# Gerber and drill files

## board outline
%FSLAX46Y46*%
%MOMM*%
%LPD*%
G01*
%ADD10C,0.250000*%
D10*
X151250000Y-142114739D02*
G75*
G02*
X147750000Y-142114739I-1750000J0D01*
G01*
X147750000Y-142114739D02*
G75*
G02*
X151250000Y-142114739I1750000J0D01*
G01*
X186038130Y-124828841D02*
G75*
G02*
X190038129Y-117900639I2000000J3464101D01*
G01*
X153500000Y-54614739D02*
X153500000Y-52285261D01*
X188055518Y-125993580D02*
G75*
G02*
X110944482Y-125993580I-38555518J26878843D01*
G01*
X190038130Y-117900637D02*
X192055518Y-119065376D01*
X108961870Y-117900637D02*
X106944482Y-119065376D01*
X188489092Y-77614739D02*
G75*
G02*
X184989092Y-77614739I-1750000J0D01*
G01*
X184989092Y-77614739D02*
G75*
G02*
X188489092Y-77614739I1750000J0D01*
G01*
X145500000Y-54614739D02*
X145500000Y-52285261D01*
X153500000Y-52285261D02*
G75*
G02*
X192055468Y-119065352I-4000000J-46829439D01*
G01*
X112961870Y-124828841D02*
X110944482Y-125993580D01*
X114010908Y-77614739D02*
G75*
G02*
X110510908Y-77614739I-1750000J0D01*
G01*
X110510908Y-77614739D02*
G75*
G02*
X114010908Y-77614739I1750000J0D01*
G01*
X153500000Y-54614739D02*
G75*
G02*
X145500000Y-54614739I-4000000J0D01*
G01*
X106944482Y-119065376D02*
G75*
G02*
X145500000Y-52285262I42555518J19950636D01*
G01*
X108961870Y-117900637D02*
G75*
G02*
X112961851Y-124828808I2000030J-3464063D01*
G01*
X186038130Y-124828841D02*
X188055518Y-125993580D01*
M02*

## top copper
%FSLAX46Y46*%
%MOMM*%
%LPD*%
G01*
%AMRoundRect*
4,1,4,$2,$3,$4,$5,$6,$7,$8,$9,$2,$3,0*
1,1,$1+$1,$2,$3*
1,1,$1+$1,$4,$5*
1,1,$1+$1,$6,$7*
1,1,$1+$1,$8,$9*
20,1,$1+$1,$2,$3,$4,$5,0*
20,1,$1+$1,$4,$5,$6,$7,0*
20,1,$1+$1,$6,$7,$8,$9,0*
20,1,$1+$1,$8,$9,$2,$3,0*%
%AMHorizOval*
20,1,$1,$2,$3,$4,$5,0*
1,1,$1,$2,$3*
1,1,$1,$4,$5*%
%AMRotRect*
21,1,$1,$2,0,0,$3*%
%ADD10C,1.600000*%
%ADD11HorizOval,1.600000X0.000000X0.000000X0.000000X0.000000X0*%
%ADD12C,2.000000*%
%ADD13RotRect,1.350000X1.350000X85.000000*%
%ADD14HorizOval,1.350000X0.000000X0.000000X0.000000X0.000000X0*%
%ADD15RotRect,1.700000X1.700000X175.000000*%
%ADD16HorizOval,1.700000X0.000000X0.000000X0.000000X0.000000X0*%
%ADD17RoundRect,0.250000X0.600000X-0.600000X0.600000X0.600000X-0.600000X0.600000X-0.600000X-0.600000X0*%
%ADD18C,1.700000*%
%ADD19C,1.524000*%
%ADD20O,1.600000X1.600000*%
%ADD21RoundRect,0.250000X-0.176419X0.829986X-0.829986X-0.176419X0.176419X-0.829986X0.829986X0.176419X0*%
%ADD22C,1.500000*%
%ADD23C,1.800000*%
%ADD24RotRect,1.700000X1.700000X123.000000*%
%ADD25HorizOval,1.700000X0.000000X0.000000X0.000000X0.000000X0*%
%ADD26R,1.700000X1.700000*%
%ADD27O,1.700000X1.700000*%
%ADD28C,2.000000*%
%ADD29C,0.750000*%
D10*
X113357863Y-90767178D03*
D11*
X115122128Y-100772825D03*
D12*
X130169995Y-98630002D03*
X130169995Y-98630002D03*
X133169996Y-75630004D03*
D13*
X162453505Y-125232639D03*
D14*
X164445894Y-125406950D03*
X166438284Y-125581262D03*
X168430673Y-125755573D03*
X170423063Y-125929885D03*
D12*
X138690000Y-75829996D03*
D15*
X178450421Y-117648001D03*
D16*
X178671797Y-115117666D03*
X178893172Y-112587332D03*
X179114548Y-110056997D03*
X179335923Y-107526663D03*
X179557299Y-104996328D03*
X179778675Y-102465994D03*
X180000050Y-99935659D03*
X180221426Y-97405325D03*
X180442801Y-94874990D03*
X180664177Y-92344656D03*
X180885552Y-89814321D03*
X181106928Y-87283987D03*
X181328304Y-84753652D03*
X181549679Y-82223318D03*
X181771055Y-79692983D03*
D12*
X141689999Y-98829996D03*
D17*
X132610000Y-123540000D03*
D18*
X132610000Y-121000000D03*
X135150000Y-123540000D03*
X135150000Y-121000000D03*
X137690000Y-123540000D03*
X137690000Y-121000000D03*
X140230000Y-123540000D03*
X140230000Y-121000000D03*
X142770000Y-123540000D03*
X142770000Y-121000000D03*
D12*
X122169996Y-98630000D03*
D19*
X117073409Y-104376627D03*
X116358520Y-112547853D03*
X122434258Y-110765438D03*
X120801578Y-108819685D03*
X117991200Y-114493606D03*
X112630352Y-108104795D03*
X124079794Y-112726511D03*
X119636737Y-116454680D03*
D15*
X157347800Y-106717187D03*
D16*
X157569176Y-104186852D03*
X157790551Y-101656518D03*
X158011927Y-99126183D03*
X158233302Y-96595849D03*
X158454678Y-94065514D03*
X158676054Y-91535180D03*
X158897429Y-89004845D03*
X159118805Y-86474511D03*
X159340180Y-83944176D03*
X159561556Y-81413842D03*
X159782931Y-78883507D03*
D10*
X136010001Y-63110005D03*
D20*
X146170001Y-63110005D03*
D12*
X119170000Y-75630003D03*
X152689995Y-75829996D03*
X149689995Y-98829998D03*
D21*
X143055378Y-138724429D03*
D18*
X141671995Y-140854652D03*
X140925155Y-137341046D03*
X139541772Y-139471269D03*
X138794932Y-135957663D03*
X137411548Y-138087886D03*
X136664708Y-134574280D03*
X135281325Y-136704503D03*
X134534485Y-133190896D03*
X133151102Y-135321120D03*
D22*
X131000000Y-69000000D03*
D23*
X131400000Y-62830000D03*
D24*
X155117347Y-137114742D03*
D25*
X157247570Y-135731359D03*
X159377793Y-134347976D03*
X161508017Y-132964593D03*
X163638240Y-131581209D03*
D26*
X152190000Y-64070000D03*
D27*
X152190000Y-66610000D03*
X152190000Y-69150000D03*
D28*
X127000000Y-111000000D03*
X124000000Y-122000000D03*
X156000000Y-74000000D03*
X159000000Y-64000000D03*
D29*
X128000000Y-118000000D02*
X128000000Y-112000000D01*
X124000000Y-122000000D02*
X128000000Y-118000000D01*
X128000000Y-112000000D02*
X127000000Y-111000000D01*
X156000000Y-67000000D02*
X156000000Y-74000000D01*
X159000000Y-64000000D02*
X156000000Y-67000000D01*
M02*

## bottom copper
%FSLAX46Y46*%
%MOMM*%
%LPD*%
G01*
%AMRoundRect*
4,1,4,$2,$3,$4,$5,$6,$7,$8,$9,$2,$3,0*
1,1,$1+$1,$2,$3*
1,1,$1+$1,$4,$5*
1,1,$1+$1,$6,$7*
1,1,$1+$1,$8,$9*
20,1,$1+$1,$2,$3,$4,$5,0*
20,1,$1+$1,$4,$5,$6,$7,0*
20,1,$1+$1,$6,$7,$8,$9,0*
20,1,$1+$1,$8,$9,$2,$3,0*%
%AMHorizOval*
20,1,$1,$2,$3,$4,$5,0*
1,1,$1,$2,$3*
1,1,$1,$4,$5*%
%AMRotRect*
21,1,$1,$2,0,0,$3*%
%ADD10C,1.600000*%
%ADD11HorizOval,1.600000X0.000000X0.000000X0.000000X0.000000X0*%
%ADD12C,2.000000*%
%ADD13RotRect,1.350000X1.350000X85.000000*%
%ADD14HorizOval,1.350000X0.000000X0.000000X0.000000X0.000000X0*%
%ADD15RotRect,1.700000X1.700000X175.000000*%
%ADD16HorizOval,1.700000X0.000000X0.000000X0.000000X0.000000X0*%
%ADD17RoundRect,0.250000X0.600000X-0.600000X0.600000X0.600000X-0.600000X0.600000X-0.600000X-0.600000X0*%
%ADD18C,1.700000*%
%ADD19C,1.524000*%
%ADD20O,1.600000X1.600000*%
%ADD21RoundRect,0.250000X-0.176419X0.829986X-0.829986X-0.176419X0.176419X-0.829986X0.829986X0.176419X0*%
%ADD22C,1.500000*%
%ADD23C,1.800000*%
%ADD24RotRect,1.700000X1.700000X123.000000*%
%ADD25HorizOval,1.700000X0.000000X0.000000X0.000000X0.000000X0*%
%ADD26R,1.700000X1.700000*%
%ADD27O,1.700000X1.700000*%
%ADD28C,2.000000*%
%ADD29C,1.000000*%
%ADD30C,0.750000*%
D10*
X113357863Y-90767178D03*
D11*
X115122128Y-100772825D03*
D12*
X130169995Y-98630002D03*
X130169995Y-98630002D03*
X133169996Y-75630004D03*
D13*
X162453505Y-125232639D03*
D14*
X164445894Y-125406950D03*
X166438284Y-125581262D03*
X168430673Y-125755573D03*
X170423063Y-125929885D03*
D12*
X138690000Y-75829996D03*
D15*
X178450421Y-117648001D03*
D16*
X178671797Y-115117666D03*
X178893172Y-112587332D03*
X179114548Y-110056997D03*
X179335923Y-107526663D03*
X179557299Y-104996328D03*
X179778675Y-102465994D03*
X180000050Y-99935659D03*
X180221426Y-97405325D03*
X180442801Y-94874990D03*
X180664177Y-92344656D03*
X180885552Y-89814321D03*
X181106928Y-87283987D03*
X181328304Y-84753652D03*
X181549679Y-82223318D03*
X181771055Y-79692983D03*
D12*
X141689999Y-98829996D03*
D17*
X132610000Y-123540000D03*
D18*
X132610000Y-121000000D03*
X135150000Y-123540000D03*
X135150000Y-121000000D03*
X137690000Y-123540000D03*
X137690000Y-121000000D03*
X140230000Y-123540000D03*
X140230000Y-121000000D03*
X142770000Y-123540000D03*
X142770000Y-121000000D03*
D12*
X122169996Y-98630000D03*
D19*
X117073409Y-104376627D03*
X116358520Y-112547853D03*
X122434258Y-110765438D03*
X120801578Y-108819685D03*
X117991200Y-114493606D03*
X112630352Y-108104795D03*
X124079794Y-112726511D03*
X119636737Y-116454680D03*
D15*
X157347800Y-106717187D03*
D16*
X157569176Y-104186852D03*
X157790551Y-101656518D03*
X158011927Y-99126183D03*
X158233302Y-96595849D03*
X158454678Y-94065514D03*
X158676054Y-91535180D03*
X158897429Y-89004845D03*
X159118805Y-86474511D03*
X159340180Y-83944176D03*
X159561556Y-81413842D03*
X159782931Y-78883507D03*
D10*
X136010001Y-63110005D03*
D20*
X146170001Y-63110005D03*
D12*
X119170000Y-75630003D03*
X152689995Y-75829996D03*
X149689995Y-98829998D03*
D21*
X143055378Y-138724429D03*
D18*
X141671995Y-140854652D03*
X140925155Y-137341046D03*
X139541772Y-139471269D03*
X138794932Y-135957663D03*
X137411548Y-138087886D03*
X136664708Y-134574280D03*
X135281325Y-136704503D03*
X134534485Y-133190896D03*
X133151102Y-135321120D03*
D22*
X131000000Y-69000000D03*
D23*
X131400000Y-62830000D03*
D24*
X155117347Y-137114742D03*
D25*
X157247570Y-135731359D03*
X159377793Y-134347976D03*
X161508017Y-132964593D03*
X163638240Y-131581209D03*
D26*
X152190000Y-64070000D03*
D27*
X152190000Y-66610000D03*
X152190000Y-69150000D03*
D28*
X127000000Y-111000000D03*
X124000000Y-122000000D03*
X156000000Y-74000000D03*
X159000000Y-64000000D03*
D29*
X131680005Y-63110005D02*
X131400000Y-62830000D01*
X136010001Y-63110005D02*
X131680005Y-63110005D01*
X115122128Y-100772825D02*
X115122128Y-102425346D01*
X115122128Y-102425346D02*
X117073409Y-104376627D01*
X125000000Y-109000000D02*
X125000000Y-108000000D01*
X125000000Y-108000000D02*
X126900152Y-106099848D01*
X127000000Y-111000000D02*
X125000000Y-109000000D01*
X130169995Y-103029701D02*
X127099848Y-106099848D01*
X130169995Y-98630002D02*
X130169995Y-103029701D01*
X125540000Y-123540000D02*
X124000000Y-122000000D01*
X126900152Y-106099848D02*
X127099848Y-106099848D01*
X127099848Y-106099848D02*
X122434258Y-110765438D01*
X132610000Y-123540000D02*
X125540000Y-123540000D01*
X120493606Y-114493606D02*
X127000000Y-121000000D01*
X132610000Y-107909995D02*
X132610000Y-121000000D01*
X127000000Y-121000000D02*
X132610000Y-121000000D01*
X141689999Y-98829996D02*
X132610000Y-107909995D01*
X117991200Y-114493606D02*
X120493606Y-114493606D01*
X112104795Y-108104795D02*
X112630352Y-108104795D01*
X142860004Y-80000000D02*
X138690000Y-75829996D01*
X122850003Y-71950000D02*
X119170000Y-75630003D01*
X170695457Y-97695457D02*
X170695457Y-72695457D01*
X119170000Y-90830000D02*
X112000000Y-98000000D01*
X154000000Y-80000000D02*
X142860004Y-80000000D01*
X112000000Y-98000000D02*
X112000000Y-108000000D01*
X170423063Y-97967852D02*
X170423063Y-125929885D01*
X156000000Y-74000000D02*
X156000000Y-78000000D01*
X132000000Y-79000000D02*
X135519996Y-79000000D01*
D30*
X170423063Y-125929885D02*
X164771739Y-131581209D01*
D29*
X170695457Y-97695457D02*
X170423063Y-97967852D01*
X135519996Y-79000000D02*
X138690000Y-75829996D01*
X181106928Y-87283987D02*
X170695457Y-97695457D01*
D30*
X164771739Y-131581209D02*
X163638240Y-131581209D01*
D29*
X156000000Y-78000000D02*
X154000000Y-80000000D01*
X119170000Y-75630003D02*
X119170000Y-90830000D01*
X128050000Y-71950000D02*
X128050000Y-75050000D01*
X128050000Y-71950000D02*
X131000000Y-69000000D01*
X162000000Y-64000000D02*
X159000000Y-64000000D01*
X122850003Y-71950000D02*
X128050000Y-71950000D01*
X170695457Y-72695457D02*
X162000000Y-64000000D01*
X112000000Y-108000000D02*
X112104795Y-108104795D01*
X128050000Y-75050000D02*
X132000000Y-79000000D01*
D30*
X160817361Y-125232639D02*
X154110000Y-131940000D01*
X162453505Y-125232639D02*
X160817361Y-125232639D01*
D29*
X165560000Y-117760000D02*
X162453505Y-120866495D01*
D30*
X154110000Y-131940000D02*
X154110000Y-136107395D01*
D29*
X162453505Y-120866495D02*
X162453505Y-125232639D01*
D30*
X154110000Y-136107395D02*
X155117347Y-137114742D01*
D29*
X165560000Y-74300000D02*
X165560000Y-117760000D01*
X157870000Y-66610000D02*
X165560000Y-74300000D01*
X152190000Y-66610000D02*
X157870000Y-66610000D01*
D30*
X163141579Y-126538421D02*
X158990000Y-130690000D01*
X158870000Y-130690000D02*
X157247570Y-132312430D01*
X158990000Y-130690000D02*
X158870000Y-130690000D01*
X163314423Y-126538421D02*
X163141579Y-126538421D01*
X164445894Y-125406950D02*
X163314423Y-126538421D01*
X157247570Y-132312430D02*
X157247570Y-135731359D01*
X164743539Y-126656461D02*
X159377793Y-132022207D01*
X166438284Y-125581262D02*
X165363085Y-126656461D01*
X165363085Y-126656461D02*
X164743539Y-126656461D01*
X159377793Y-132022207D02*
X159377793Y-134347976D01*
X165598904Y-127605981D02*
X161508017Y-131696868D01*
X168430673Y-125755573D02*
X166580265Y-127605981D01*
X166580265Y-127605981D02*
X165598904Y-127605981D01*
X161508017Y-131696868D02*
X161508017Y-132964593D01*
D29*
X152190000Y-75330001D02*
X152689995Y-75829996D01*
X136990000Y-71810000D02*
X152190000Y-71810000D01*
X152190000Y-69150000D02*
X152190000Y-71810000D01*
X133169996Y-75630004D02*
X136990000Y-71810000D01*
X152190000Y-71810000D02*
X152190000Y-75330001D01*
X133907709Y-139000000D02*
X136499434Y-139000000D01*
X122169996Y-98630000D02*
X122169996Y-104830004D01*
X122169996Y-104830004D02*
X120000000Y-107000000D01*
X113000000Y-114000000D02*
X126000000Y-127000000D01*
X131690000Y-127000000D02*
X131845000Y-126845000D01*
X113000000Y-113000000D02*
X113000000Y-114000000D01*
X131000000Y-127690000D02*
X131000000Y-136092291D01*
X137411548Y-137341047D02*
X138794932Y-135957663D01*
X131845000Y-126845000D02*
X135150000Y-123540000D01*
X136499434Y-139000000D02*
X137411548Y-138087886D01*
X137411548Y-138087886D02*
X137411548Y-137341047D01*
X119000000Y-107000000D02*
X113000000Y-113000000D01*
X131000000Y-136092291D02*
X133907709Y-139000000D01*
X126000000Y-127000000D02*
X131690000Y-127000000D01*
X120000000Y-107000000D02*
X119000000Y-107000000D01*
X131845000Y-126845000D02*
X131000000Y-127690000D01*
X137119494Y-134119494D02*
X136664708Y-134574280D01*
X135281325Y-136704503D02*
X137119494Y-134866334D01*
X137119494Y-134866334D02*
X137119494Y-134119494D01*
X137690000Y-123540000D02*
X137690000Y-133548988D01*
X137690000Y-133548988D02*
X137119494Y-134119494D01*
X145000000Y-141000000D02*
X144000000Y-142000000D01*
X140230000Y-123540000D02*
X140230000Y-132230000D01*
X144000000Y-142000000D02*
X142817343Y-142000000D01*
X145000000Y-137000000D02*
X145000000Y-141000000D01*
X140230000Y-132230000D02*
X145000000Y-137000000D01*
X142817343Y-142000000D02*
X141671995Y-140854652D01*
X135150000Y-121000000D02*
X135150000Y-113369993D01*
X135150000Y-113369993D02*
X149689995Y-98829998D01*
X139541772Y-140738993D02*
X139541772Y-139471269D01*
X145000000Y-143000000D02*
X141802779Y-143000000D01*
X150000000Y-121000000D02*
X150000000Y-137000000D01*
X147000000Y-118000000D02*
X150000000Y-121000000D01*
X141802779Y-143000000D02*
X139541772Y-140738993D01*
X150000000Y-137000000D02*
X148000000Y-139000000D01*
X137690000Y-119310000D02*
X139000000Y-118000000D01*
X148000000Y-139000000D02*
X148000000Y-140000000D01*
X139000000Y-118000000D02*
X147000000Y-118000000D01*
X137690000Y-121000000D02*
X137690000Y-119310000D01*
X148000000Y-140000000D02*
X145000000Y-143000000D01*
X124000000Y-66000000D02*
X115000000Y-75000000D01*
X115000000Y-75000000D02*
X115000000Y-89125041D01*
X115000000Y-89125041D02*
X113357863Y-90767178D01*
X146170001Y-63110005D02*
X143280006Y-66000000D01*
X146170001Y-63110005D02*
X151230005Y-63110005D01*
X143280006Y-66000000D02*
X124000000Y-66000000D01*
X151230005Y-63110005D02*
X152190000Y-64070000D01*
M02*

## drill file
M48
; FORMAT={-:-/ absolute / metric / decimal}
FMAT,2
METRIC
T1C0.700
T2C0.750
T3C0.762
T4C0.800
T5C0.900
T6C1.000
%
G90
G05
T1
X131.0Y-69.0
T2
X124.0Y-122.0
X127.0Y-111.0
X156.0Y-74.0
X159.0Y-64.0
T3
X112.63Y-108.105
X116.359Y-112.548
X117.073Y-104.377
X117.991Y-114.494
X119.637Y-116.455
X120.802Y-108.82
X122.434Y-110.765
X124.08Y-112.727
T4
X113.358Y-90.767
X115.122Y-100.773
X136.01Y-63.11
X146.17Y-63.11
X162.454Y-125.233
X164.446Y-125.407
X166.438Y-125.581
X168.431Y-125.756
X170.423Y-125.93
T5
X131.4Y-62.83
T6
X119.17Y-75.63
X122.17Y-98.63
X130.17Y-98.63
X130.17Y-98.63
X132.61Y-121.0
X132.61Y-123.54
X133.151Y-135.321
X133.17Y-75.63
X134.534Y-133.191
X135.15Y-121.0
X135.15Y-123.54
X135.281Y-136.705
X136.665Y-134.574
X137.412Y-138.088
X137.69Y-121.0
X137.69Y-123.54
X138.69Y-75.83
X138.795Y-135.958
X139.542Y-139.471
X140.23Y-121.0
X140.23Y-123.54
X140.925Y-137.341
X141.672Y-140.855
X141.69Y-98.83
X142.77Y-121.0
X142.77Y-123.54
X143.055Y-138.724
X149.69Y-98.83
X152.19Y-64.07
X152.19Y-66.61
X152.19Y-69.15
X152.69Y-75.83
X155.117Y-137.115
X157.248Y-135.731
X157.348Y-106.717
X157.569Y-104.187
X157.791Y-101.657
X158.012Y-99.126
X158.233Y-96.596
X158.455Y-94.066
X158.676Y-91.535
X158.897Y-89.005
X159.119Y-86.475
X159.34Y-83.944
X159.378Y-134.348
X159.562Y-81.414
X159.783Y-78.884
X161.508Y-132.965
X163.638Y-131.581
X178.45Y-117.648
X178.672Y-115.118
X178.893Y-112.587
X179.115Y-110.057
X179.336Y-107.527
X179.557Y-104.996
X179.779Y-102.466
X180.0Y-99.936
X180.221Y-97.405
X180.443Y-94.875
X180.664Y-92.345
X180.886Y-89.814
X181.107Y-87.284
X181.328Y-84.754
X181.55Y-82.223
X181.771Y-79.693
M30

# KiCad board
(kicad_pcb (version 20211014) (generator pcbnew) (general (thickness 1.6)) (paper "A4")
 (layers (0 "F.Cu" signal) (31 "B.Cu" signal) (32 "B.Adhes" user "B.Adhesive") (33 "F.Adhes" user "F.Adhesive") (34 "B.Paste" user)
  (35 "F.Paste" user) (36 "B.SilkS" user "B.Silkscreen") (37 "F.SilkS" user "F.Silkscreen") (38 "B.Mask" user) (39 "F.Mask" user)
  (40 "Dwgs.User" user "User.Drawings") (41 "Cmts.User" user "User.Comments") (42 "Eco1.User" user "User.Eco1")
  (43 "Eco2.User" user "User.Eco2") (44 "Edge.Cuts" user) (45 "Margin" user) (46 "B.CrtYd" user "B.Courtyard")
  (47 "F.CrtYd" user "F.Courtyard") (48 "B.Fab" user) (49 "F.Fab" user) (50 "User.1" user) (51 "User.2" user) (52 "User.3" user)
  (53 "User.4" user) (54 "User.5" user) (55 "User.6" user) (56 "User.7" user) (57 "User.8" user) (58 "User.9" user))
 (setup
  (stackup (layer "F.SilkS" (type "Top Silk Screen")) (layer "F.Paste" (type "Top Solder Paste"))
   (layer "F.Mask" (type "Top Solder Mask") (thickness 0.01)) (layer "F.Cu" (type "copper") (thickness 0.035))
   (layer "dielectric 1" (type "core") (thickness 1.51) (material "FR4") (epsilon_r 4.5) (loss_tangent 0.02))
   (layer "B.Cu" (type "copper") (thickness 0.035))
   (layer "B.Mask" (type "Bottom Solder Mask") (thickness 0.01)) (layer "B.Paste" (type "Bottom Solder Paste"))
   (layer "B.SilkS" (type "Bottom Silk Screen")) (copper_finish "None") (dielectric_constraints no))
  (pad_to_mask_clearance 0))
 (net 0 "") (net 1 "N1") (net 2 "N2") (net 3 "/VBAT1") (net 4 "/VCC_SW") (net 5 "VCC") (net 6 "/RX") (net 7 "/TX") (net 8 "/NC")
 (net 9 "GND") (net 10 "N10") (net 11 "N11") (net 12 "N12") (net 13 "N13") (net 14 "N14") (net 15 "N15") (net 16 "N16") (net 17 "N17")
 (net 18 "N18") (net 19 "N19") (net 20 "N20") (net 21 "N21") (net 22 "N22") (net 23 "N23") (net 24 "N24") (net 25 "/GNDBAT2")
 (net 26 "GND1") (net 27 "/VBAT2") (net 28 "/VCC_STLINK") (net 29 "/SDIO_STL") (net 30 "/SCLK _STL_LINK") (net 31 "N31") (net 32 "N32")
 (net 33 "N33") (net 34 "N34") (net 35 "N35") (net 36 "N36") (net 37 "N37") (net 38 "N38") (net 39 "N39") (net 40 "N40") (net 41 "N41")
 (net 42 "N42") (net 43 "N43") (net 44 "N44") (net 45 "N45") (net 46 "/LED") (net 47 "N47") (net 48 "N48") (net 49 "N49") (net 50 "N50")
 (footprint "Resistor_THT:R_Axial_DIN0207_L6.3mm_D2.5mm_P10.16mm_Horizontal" (layer "F.Cu") (at 113.357863 90.767178 -80)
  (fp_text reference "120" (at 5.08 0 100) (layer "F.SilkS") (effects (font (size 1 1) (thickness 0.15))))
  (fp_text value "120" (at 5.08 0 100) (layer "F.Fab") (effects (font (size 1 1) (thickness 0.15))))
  (pad "1" thru_hole circle locked (at 0 0 280) (size 1.6 1.6) (drill 0.8) (layers *.Cu *.Mask) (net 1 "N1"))
  (pad "2" thru_hole oval locked (at 10.16 0 280) (size 1.6 1.6) (drill 0.8) (layers *.Cu *.Mask) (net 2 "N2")))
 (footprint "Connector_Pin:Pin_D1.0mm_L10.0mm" (layer "F.Cu") (at 130.169995 98.630002 90)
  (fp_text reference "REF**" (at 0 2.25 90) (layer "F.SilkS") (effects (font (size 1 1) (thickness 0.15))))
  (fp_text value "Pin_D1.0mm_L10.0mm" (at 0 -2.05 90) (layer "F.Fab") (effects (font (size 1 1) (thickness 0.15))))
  (pad "1" thru_hole circle locked (at 0 0 90) (size 2 2) (drill 1) (layers *.Cu *.Mask) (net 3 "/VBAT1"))
  (pad "1" thru_hole circle locked (at 0 0 90) (size 2 2) (drill 1) (layers *.Cu *.Mask) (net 3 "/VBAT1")))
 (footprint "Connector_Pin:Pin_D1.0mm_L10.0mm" (layer "F.Cu") (at 133.169996 75.630004 90)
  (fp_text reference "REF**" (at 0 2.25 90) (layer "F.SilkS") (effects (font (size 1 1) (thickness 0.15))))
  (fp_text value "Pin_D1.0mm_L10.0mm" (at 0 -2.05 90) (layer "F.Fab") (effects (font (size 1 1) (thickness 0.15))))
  (pad "1" thru_hole circle locked (at 0 0 90) (size 2 2) (drill 1) (layers *.Cu *.Mask) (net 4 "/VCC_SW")))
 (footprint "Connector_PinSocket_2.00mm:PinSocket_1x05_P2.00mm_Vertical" (layer "F.Cu") (at 162.453505 125.232639 85)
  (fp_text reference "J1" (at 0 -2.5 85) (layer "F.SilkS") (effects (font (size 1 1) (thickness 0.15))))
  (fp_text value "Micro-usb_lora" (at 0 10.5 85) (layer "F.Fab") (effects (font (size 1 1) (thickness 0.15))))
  (pad "1" thru_hole rect locked (at 0 0 85) (size 1.35 1.35) (drill 0.8) (layers *.Cu *.Mask) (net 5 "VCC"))
  (pad "2" thru_hole oval locked (at 0 2 85) (size 1.35 1.35) (drill 0.8) (layers *.Cu *.Mask) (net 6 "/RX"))
  (pad "3" thru_hole oval locked (at 0 4 85) (size 1.35 1.35) (drill 0.8) (layers *.Cu *.Mask) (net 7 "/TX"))
  (pad "4" thru_hole oval locked (at 0 6 85) (size 1.35 1.35) (drill 0.8) (layers *.Cu *.Mask) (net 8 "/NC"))
  (pad "5" thru_hole oval locked (at 0 8 85) (size 1.35 1.35) (drill 0.8) (layers *.Cu *.Mask) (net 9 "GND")))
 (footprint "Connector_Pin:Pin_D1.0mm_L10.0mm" (layer "F.Cu") (at 138.69 75.829996 90)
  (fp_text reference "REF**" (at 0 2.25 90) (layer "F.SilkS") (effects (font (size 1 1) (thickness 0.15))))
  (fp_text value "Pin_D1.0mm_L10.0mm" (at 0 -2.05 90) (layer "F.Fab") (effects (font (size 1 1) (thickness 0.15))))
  (pad "1" thru_hole circle locked (at 0 0 90) (size 2 2) (drill 1) (layers *.Cu *.Mask) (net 9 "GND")))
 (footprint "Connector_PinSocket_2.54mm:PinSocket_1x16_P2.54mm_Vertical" (layer "F.Cu") (at 178.450421 117.648001 175)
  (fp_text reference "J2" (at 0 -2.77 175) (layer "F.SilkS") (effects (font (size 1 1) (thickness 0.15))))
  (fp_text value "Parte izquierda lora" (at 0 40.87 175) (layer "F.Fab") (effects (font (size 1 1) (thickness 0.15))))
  (pad "1" thru_hole rect locked (at 0 0 175) (size 1.7 1.7) (drill 1) (layers *.Cu *.Mask) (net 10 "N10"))
  (pad "2" thru_hole oval locked (at 0 2.54 175) (size 1.7 1.7) (drill 1) (layers *.Cu *.Mask) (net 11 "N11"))
  (pad "3" thru_hole oval locked (at 0 5.08 175) (size 1.7 1.7) (drill 1) (layers *.Cu *.Mask) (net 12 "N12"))
  (pad "4" thru_hole oval locked (at 0 7.62 175) (size 1.7 1.7) (drill 1) (layers *.Cu *.Mask) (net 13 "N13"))
  (pad "5" thru_hole oval locked (at 0 10.16 175) (size 1.7 1.7) (drill 1) (layers *.Cu *.Mask) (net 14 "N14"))
  (pad "6" thru_hole oval locked (at 0 12.7 175) (size 1.7 1.7) (drill 1) (layers *.Cu *.Mask) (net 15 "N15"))
  (pad "7" thru_hole oval locked (at 0 15.24 175) (size 1.7 1.7) (drill 1) (layers *.Cu *.Mask) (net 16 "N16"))
  (pad "8" thru_hole oval locked (at 0 17.78 175) (size 1.7 1.7) (drill 1) (layers *.Cu *.Mask) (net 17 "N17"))
  (pad "9" thru_hole oval locked (at 0 20.32 175) (size 1.7 1.7) (drill 1) (layers *.Cu *.Mask) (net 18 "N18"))
  (pad "10" thru_hole oval locked (at 0 22.86 175) (size 1.7 1.7) (drill 1) (layers *.Cu *.Mask) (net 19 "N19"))
  (pad "11" thru_hole oval locked (at 0 25.4 175) (size 1.7 1.7) (drill 1) (layers *.Cu *.Mask) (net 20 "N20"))
  (pad "12" thru_hole oval locked (at 0 27.94 175) (size 1.7 1.7) (drill 1) (layers *.Cu *.Mask) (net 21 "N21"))
  (pad "13" thru_hole oval locked (at 0 30.48 175) (size 1.7 1.7) (drill 1) (layers *.Cu *.Mask) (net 9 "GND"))
  (pad "14" thru_hole oval locked (at 0 33.02 175) (size 1.7 1.7) (drill 1) (layers *.Cu *.Mask) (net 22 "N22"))
  (pad "15" thru_hole oval locked (at 0 35.56 175) (size 1.7 1.7) (drill 1) (layers *.Cu *.Mask) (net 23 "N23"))
  (pad "16" thru_hole oval locked (at 0 38.1 175) (size 1.7 1.7) (drill 1) (layers *.Cu *.Mask) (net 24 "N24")))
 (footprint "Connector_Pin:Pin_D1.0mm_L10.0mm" (layer "F.Cu") (at 141.689999 98.829996 90)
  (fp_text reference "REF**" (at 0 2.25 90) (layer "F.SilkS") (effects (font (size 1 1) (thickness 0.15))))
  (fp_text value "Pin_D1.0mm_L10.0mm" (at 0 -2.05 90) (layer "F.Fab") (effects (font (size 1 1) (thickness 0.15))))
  (pad "1" thru_hole circle locked (at 0 0 90) (size 2 2) (drill 1) (layers *.Cu *.Mask) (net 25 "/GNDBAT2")))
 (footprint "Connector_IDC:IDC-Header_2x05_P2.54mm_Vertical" (layer "F.Cu") (at 132.61 123.54 90)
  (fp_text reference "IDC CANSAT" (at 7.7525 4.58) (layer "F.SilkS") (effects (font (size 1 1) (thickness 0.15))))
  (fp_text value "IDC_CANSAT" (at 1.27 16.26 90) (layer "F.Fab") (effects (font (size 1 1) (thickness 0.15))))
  (pad "1" thru_hole roundrect locked (at 0 0 90) (size 1.7 1.7) (drill 1) (layers *.Cu *.Mask) (roundrect_rratio 0.147059) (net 3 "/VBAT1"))
  (pad "2" thru_hole circle locked (at 2.54 0 90) (size 1.7 1.7) (drill 1) (layers *.Cu *.Mask) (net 25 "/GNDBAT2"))
  (pad "3" thru_hole circle locked (at 0 2.54 90) (size 1.7 1.7) (drill 1) (layers *.Cu *.Mask) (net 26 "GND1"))
  (pad "4" thru_hole circle locked (at 2.54 2.54 90) (size 1.7 1.7) (drill 1) (layers *.Cu *.Mask) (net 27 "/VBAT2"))
  (pad "5" thru_hole circle locked (at 0 5.08 90) (size 1.7 1.7) (drill 1) (layers *.Cu *.Mask) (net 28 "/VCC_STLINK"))
  (pad "6" thru_hole circle locked (at 2.54 5.08 90) (size 1.7 1.7) (drill 1) (layers *.Cu *.Mask) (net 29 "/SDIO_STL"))
  (pad "7" thru_hole circle locked (at 0 7.62 90) (size 1.7 1.7) (drill 1) (layers *.Cu *.Mask) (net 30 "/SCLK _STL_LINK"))
  (pad "8" thru_hole circle locked (at 2.54 7.62 90) (size 1.7 1.7) (drill 1) (layers *.Cu *.Mask) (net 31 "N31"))
  (pad "9" thru_hole circle locked (at 0 10.16 90) (size 1.7 1.7) (drill 1) (layers *.Cu *.Mask) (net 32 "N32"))
  (pad "10" thru_hole circle locked (at 2.54 10.16 90) (size 1.7 1.7) (drill 1) (layers *.Cu *.Mask) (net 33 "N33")))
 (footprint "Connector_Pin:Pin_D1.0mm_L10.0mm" (layer "F.Cu") (at 122.169996 98.63 90)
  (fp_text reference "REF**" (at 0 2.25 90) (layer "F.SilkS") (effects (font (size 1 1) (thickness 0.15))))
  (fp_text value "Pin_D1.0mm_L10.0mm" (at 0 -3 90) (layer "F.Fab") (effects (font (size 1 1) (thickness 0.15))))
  (pad "1" thru_hole circle locked (at 0 0 90) (size 2 2) (drill 1) (layers *.Cu *.Mask) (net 26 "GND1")))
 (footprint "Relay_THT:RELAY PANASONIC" (layer "F.Cu") (at 119.03 111.22 -50)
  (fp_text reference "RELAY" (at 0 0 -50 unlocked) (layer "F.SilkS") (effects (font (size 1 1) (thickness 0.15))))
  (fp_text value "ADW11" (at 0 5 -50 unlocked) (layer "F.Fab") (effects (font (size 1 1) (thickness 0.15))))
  (pad "1" thru_hole circle (at -6.5 -2.9 310) (size 1.524 1.524) (drill 0.762) (layers *.Cu *.Mask) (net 2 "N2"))
  (pad "2" thru_hole circle (at -0.7 2.9 310) (size 1.524 1.524) (drill 0.762) (layers *.Cu *.Mask))
  (pad "3" thru_hole circle (at 1.84 -2.9 310) (size 1.524 1.524) (drill 0.762) (layers *.Cu *.Mask) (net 3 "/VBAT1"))
  (pad "4" thru_hole circle (at -0.7 -2.9 310) (size 1.524 1.524) (drill 0.762) (layers *.Cu *.Mask))
  (pad "5" thru_hole circle (at 1.84 2.9 310) (size 1.524 1.524) (drill 0.762) (layers *.Cu *.Mask) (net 25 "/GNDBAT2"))
  (pad "6" thru_hole circle (at -6.5 2.9 310) (size 1.524 1.524) (drill 0.762) (layers *.Cu *.Mask) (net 9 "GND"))
  (pad "7" thru_hole circle (at 4.4 -2.9 310) (size 1.524 1.524) (drill 0.762) (layers *.Cu *.Mask))
  (pad "8" thru_hole circle (at 4.4 2.9 310) (size 1.524 1.524) (drill 0.762) (layers *.Cu *.Mask)))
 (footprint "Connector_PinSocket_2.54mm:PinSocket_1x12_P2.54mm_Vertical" (layer "F.Cu") (at 157.3478 106.717187 175)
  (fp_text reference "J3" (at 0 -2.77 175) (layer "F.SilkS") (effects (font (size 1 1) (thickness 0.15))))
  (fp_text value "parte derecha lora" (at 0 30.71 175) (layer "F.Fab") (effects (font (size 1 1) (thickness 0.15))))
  (pad "1" thru_hole rect locked (at 0 0 175) (size 1.7 1.7) (drill 1) (layers *.Cu *.Mask) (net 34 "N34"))
  (pad "2" thru_hole oval locked (at 0 2.54 175) (size 1.7 1.7) (drill 1) (layers *.Cu *.Mask) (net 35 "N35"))
  (pad "3" thru_hole oval locked (at 0 5.08 175) (size 1.7 1.7) (drill 1) (layers *.Cu *.Mask) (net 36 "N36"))
  (pad "4" thru_hole oval locked (at 0 7.62 175) (size 1.7 1.7) (drill 1) (layers *.Cu *.Mask) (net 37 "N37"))
  (pad "5" thru_hole oval locked (at 0 10.16 175) (size 1.7 1.7) (drill 1) (layers *.Cu *.Mask) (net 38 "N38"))
  (pad "6" thru_hole oval locked (at 0 12.7 175) (size 1.7 1.7) (drill 1) (layers *.Cu *.Mask) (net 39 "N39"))
  (pad "7" thru_hole oval locked (at 0 15.24 175) (size 1.7 1.7) (drill 1) (layers *.Cu *.Mask) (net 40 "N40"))
  (pad "8" thru_hole oval locked (at 0 17.78 175) (size 1.7 1.7) (drill 1) (layers *.Cu *.Mask) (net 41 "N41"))
  (pad "9" thru_hole oval locked (at 0 20.32 175) (size 1.7 1.7) (drill 1) (layers *.Cu *.Mask) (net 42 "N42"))
  (pad "10" thru_hole oval locked (at 0 22.86 175) (size 1.7 1.7) (drill 1) (layers *.Cu *.Mask) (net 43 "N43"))
  (pad "11" thru_hole oval locked (at 0 25.4 175) (size 1.7 1.7) (drill 1) (layers *.Cu *.Mask) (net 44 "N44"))
  (pad "12" thru_hole oval locked (at 0 27.94 175) (size 1.7 1.7) (drill 1) (layers *.Cu *.Mask) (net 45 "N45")))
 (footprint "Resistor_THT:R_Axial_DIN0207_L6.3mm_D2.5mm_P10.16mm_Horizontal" (layer "F.Cu") (at 136.010001 63.110005)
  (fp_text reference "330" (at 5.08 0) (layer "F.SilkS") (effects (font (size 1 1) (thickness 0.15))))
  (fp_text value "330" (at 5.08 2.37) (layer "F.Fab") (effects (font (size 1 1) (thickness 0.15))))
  (pad "1" thru_hole circle locked (at 0 0) (size 1.6 1.6) (drill 0.8) (layers *.Cu *.Mask) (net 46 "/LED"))
  (pad "2" thru_hole oval locked (at 10.16 0) (size 1.6 1.6) (drill 0.8) (layers *.Cu *.Mask) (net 1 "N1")))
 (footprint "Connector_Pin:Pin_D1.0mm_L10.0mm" (layer "F.Cu") (at 119.17 75.630003 90)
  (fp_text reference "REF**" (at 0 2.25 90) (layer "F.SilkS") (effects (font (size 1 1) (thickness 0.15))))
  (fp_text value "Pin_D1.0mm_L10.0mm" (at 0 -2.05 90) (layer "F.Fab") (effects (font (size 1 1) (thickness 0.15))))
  (pad "1" thru_hole circle locked (at 0 0 90) (size 2 2) (drill 1) (layers *.Cu *.Mask) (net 9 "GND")))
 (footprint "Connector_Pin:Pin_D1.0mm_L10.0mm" (layer "F.Cu") (at 152.689995 75.829996 90)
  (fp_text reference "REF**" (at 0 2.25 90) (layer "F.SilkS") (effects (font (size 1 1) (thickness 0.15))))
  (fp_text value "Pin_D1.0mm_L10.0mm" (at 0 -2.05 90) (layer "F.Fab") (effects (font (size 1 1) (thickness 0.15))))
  (pad "1" thru_hole circle locked (at 0 0 90) (size 2 2) (drill 1) (layers *.Cu *.Mask) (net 4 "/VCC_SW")))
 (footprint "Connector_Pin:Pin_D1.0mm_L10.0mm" (layer "F.Cu") (at 149.689995 98.829998 90)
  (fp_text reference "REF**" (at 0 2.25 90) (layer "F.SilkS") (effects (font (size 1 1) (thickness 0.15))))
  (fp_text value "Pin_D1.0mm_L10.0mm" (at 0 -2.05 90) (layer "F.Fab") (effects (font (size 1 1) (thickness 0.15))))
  (pad "1" thru_hole circle locked (at 0 0 90) (size 2 2) (drill 1) (layers *.Cu *.Mask) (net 27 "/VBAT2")))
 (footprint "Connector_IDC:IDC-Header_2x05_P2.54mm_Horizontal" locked (layer "F.Cu") (at 143.055378 138.724429 -123)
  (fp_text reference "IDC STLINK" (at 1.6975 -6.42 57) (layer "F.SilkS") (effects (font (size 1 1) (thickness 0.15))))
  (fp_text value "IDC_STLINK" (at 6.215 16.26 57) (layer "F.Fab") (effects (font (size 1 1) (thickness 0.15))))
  (pad "1" thru_hole roundrect locked (at 0 0 237) (size 1.7 1.7) (drill 1) (layers *.Cu *.Mask) (roundrect_rratio 0.147059) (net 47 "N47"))
  (pad "2" thru_hole circle locked (at 2.54 0 237) (size 1.7 1.7) (drill 1) (layers *.Cu *.Mask) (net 30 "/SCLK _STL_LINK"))
  (pad "3" thru_hole circle locked (at 0 2.54 237) (size 1.7 1.7) (drill 1) (layers *.Cu *.Mask) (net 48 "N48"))
  (pad "4" thru_hole circle locked (at 2.54 2.54 237) (size 1.7 1.7) (drill 1) (layers *.Cu *.Mask) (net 29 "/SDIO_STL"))
  (pad "5" thru_hole circle locked (at 0 5.08 237) (size 1.7 1.7) (drill 1) (layers *.Cu *.Mask) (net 26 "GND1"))
  (pad "6" thru_hole circle locked (at 2.54 5.08 237) (size 1.7 1.7) (drill 1) (layers *.Cu *.Mask) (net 26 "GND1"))
  (pad "7" thru_hole circle locked (at 0 7.62 237) (size 1.7 1.7) (drill 1) (layers *.Cu *.Mask) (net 28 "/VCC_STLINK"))
  (pad "8" thru_hole circle locked (at 2.54 7.62 237) (size 1.7 1.7) (drill 1) (layers *.Cu *.Mask) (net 28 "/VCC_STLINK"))
  (pad "9" thru_hole circle locked (at 0 10.16 237) (size 1.7 1.7) (drill 1) (layers *.Cu *.Mask) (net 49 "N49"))
  (pad "10" thru_hole circle locked (at 2.54 10.16 237) (size 1.7 1.7) (drill 1) (layers *.Cu *.Mask) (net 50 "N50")))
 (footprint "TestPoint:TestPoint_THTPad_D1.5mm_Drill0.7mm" (layer "F.Cu") (at 131 69 -10)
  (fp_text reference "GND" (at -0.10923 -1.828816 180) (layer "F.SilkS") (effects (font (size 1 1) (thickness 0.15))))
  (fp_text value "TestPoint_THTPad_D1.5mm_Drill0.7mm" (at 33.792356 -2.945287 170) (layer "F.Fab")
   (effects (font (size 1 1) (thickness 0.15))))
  (pad "1" thru_hole circle locked (at 0 0 350) (size 1.5 1.5) (drill 0.7) (layers *.Cu *.Mask) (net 9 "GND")))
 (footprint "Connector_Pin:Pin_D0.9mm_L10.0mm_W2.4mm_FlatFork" (layer "F.Cu") (at 131.4 62.83 90)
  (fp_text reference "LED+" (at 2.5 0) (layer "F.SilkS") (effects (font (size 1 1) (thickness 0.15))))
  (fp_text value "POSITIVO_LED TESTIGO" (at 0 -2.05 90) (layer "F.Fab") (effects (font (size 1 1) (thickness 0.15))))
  (pad "1" thru_hole circle locked (at 0 0 90) (size 1.8 1.8) (drill 0.9) (layers *.Cu *.Mask) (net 46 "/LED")))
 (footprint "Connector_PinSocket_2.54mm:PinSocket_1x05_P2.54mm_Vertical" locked (layer "F.Cu") (at 155.117347 137.114742 123)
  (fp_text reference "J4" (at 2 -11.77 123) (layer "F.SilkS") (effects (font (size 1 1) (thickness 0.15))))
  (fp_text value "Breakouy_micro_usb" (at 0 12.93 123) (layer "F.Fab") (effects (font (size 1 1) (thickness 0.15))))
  (pad "1" thru_hole rect locked (at 0 0 123) (size 1.7 1.7) (drill 1) (layers *.Cu *.Mask) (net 5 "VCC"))
  (pad "2" thru_hole oval locked (at 0 2.54 123) (size 1.7 1.7) (drill 1) (layers *.Cu *.Mask) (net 6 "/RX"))
  (pad "3" thru_hole oval locked (at 0 5.08 123) (size 1.7 1.7) (drill 1) (layers *.Cu *.Mask) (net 7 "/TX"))
  (pad "4" thru_hole oval locked (at 0 7.62 123) (size 1.7 1.7) (drill 1) (layers *.Cu *.Mask) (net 8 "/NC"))
  (pad "5" thru_hole oval locked (at 0 10.16 123) (size 1.7 1.7) (drill 1) (layers *.Cu *.Mask) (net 9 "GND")))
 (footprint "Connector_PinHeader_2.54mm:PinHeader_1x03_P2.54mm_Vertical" (layer "F.Cu") (at 152.19 64.07)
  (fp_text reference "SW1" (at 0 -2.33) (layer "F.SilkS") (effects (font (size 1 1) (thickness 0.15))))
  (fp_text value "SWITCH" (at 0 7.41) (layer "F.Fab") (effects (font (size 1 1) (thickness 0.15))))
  (pad "1" thru_hole rect locked (at 0 0) (size 1.7 1.7) (drill 1) (layers *.Cu *.Mask) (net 1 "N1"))
  (pad "2" thru_hole oval locked (at 0 2.54) (size 1.7 1.7) (drill 1) (layers *.Cu *.Mask) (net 5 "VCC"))
  (pad "3" thru_hole oval locked (at 0 5.08) (size 1.7 1.7) (drill 1) (layers *.Cu *.Mask) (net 4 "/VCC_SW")))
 (gr_circle (center 149.5 142.114739) (end 151.25 142.114739) (layer "Edge.Cuts") (width 0.25) (fill none))
 (gr_arc (start 186.03813 124.828841) (mid 184.574029 119.364739) (end 190.03813 117.900637) (layer "Edge.Cuts") (width 0.25))
 (gr_line (start 153.5 54.614739) (end 153.5 52.285261) (layer "Edge.Cuts") (width 0.25))
 (gr_arc (start 188.055518 125.99358) (mid 149.5 146.114739) (end 110.944482 125.99358) (layer "Edge.Cuts") (width 0.25))
 (gr_line (start 190.03813 117.900637) (end 192.055518 119.065376) (layer "Edge.Cuts") (width 0.25))
 (gr_line (start 108.96187 117.900637) (end 106.944482 119.065376) (layer "Edge.Cuts") (width 0.25))
 (gr_circle (center 186.739092 77.614739) (end 188.489092 77.614739) (layer "Edge.Cuts") (width 0.25) (fill none))
 (gr_line (start 145.5 54.614739) (end 145.5 52.285261) (layer "Edge.Cuts") (width 0.25))
 (gr_arc (start 153.5 52.285261) (mid 190.203194 75.614739) (end 192.055518 119.065376) (layer "Edge.Cuts") (width 0.25))
 (gr_line (start 112.96187 124.828841) (end 110.944482 125.99358) (layer "Edge.Cuts") (width 0.25))
 (gr_circle (center 112.260908 77.614739) (end 114.010908 77.614739) (layer "Edge.Cuts") (width 0.25) (fill none))
 (gr_arc (start 153.5 54.614739) (mid 149.5 58.614739) (end 145.5 54.614739) (layer "Edge.Cuts") (width 0.25))
 (gr_arc (start 106.944482 119.065376) (mid 108.796806 75.614739) (end 145.5 52.285261) (layer "Edge.Cuts") (width 0.25))
 (gr_arc (start 108.96187 117.900637) (mid 114.425971 119.364739) (end 112.96187 124.828841) (layer "Edge.Cuts") (width 0.25))
 (gr_line (start 186.03813 124.828841) (end 188.055518 125.99358) (layer "Edge.Cuts") (width 0.25))
 (segment (start 131.680005 63.110005) (end 131.4 62.83) (width 1) (layer "B.Cu") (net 46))
 (segment (start 136.010001 63.110005) (end 131.680005 63.110005) (width 1) (layer "B.Cu") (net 46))
 (segment (start 115.122128 100.772825) (end 115.122128 102.425346) (width 1) (layer "B.Cu") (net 2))
 (segment (start 115.122128 102.425346) (end 117.073409 104.376627) (width 1) (layer "B.Cu") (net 2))
 (segment (start 128 118) (end 128 112) (width 0.75) (layer "F.Cu") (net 3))
 (segment (start 124 122) (end 128 118) (width 0.75) (layer "F.Cu") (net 3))
 (segment (start 128 112) (end 127 111) (width 0.75) (layer "F.Cu") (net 3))
 (via (at 127 111) (size 2) (drill 0.75) (layers "F.Cu" "B.Cu") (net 3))
 (via (at 124 122) (size 2) (drill 0.75) (layers "F.Cu" "B.Cu") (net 3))
 (segment (start 125 109) (end 125 108) (width 1) (layer "B.Cu") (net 3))
 (segment (start 125 108) (end 126.900152 106.099848) (width 1) (layer "B.Cu") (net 3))
 (segment (start 127 111) (end 125 109) (width 1) (layer "B.Cu") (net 3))
 (segment (start 130.169995 103.029701) (end 127.099848 106.099848) (width 1) (layer "B.Cu") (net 3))
 (segment (start 130.169995 98.630002) (end 130.169995 103.029701) (width 1) (layer "B.Cu") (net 3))
 (segment (start 125.54 123.54) (end 124 122) (width 1) (layer "B.Cu") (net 3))
 (segment (start 126.900152 106.099848) (end 127.099848 106.099848) (width 1) (layer "B.Cu") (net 3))
 (segment (start 127.099848 106.099848) (end 122.434258 110.765438) (width 1) (layer "B.Cu") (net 3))
 (segment (start 132.61 123.54) (end 125.54 123.54) (width 1) (layer "B.Cu") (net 3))
 (segment (start 120.493606 114.493606) (end 127 121) (width 1) (layer "B.Cu") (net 25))
 (segment (start 132.61 107.909995) (end 132.61 121) (width 1) (layer "B.Cu") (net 25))
 (segment (start 127 121) (end 132.61 121) (width 1) (layer "B.Cu") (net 25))
 (segment (start 141.689999 98.829996) (end 132.61 107.909995) (width 1) (layer "B.Cu") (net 25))
 (segment (start 117.9912 114.493606) (end 120.493606 114.493606) (width 1) (layer "B.Cu") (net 25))
 (segment (start 156 67) (end 156 74) (width 0.75) (layer "F.Cu") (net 9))
 (segment (start 159 64) (end 156 67) (width 0.75) (layer "F.Cu") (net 9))
 (via (at 156 74) (size 2) (drill 0.75) (layers "F.Cu" "B.Cu") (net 9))
 (via (at 159 64) (size 2) (drill 0.75) (layers "F.Cu" "B.Cu") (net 9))
 (segment (start 112.104795 108.104795) (end 112.630352 108.104795) (width 1) (layer "B.Cu") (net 9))
 (segment (start 142.860004 80) (end 138.69 75.829996) (width 1) (layer "B.Cu") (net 9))
 (segment (start 122.850003 71.95) (end 119.17 75.630003) (width 1) (layer "B.Cu") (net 9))
 (segment (start 170.695457 97.695457) (end 170.695457 72.695457) (width 1) (layer "B.Cu") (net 9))
 (segment (start 119.17 90.83) (end 112 98) (width 1) (layer "B.Cu") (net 9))
 (segment (start 154 80) (end 142.860004 80) (width 1) (layer "B.Cu") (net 9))
 (segment (start 112 98) (end 112 108) (width 1) (layer "B.Cu") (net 9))
 (segment (start 170.423063 97.967852) (end 170.423063 125.929885) (width 1) (layer "B.Cu") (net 9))
 (segment (start 156 74) (end 156 78) (width 1) (layer "B.Cu") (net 9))
 (segment (start 132 79) (end 135.519996 79) (width 1) (layer "B.Cu") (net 9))
 (segment (start 170.423063 125.929885) (end 164.771739 131.581209) (width 0.75) (layer "B.Cu") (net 9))
 (segment (start 170.695457 97.695457) (end 170.423063 97.967852) (width 1) (layer "B.Cu") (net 9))
 (segment (start 135.519996 79) (end 138.69 75.829996) (width 1) (layer "B.Cu") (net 9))
 (segment (start 181.106928 87.283987) (end 170.695457 97.695457) (width 1) (layer "B.Cu") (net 9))
 (segment (start 164.771739 131.581209) (end 163.63824 131.581209) (width 0.75) (layer "B.Cu") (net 9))
 (segment (start 156 78) (end 154 80) (width 1) (layer "B.Cu") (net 9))
 (segment (start 119.17 75.630003) (end 119.17 90.83) (width 1) (layer "B.Cu") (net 9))
 (segment (start 128.05 71.95) (end 128.05 75.05) (width 1) (layer "B.Cu") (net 9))
 (segment (start 128.05 71.95) (end 131 69) (width 1) (layer "B.Cu") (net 9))
 (segment (start 162 64) (end 159 64) (width 1) (layer "B.Cu") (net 9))
 (segment (start 122.850003 71.95) (end 128.05 71.95) (width 1) (layer "B.Cu") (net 9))
 (segment (start 170.695457 72.695457) (end 162 64) (width 1) (layer "B.Cu") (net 9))
 (segment (start 112 108) (end 112.104795 108.104795) (width 1) (layer "B.Cu") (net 9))
 (segment (start 128.05 75.05) (end 132 79) (width 1) (layer "B.Cu") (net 9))
 (segment (start 160.817361 125.232639) (end 154.11 131.94) (width 0.75) (layer "B.Cu") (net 5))
 (segment (start 162.453505 125.232639) (end 160.817361 125.232639) (width 0.75) (layer "B.Cu") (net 5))
 (segment (start 165.56 117.76) (end 162.453505 120.866495) (width 1) (layer "B.Cu") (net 5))
 (segment (start 154.11 131.94) (end 154.11 136.107395) (width 0.75) (layer "B.Cu") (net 5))
 (segment (start 162.453505 120.866495) (end 162.453505 125.232639) (width 1) (layer "B.Cu") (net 5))
 (segment (start 154.11 136.107395) (end 155.117347 137.114742) (width 0.75) (layer "B.Cu") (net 5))
 (segment (start 165.56 74.3) (end 165.56 117.76) (width 1) (layer "B.Cu") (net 5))
 (segment (start 157.87 66.61) (end 165.56 74.3) (width 1) (layer "B.Cu") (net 5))
 (segment (start 152.19 66.61) (end 157.87 66.61) (width 1) (layer "B.Cu") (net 5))
 (segment (start 163.141579 126.538421) (end 158.99 130.69) (width 0.75) (layer "B.Cu") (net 6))
 (segment (start 158.87 130.69) (end 157.24757 132.31243) (width 0.75) (layer "B.Cu") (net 6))
 (segment (start 158.99 130.69) (end 158.87 130.69) (width 0.75) (layer "B.Cu") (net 6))
 (segment (start 163.314423 126.538421) (end 163.141579 126.538421) (width 0.75) (layer "B.Cu") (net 6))
 (segment (start 164.445894 125.40695) (end 163.314423 126.538421) (width 0.75) (layer "B.Cu") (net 6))
 (segment (start 157.24757 132.31243) (end 157.24757 135.731359) (width 0.75) (layer "B.Cu") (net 6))
 (segment (start 164.743539 126.656461) (end 159.377793 132.022207) (width 0.75) (layer "B.Cu") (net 7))
 (segment (start 166.438284 125.581262) (end 165.363085 126.656461) (width 0.75) (layer "B.Cu") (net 7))
 (segment (start 165.363085 126.656461) (end 164.743539 126.656461) (width 0.75) (layer "B.Cu") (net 7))
 (segment (start 159.377793 132.022207) (end 159.377793 134.347976) (width 0.75) (layer "B.Cu") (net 7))
 (segment (start 165.598904 127.605981) (end 161.508017 131.696868) (width 0.75) (layer "B.Cu") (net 8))
 (segment (start 168.430673 125.755573) (end 166.580265 127.605981) (width 0.75) (layer "B.Cu") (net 8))
 (segment (start 166.580265 127.605981) (end 165.598904 127.605981) (width 0.75) (layer "B.Cu") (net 8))
 (segment (start 161.508017 131.696868) (end 161.508017 132.964593) (width 0.75) (layer "B.Cu") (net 8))
 (segment (start 152.19 75.330001) (end 152.689995 75.829996) (width 1) (layer "B.Cu") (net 4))
 (segment (start 136.99 71.81) (end 152.19 71.81) (width 1) (layer "B.Cu") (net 4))
 (segment (start 152.19 69.15) (end 152.19 71.81) (width 1) (layer "B.Cu") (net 4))
 (segment (start 133.169996 75.630004) (end 136.99 71.81) (width 1) (layer "B.Cu") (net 4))
 (segment (start 152.19 71.81) (end 152.19 75.330001) (width 1) (layer "B.Cu") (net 4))
 (segment (start 133.907709 139) (end 136.499434 139) (width 1) (layer "B.Cu") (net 26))
 (segment (start 122.169996 98.63) (end 122.169996 104.830004) (width 1) (layer "B.Cu") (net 26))
 (segment (start 122.169996 104.830004) (end 120 107) (width 1) (layer "B.Cu") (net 26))
 (segment (start 113 114) (end 126 127) (width 1) (layer "B.Cu") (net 26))
 (segment (start 131.69 127) (end 131.845 126.845) (width 1) (layer "B.Cu") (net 26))
 (segment (start 113 113) (end 113 114) (width 1) (layer "B.Cu") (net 26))
 (segment (start 131 127.69) (end 131 136.092291) (width 1) (layer "B.Cu") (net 26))
 (segment (start 137.411548 137.341047) (end 138.794932 135.957663) (width 1) (layer "B.Cu") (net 26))
 (segment (start 131.845 126.845) (end 135.15 123.54) (width 1) (layer "B.Cu") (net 26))
 (segment (start 136.499434 139) (end 137.411548 138.087886) (width 1) (layer "B.Cu") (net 26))
 (segment (start 137.411548 138.087886) (end 137.411548 137.341047) (width 1) (layer "B.Cu") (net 26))
 (segment (start 119 107) (end 113 113) (width 1) (layer "B.Cu") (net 26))
 (segment (start 131 136.092291) (end 133.907709 139) (width 1) (layer "B.Cu") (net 26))
 (segment (start 126 127) (end 131.69 127) (width 1) (layer "B.Cu") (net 26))
 (segment (start 120 107) (end 119 107) (width 1) (layer "B.Cu") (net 26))
 (segment (start 131.845 126.845) (end 131 127.69) (width 1) (layer "B.Cu") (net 26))
 (segment (start 137.119494 134.119494) (end 136.664708 134.57428) (width 1) (layer "B.Cu") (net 28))
 (segment (start 135.281325 136.704503) (end 137.119494 134.866334) (width 1) (layer "B.Cu") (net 28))
 (segment (start 137.119494 134.866334) (end 137.119494 134.119494) (width 1) (layer "B.Cu") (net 28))
 (segment (start 137.69 123.54) (end 137.69 133.548988) (width 1) (layer "B.Cu") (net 28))
 (segment (start 137.69 133.548988) (end 137.119494 134.119494) (width 1) (layer "B.Cu") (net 28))
 (segment (start 145 141) (end 144 142) (width 1) (layer "B.Cu") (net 30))
 (segment (start 140.23 123.54) (end 140.23 132.23) (width 1) (layer "B.Cu") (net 30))
 (segment (start 144 142) (end 142.817343 142) (width 1) (layer "B.Cu") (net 30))
 (segment (start 145 137) (end 145 141) (width 1) (layer "B.Cu") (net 30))
 (segment (start 140.23 132.23) (end 145 137) (width 1) (layer "B.Cu") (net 30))
 (segment (start 142.817343 142) (end 141.671995 140.854652) (width 1) (layer "B.Cu") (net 30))
 (segment (start 135.15 121) (end 135.15 113.369993) (width 1) (layer "B.Cu") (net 27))
 (segment (start 135.15 113.369993) (end 149.689995 98.829998) (width 1) (layer "B.Cu") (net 27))
 (segment (start 139.541772 140.738993) (end 139.541772 139.471269) (width 1) (layer "B.Cu") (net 29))
 (segment (start 145 143) (end 141.802779 143) (width 1) (layer "B.Cu") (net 29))
 (segment (start 150 121) (end 150 137) (width 1) (layer "B.Cu") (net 29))
 (segment (start 147 118) (end 150 121) (width 1) (layer "B.Cu") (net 29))
 (segment (start 141.802779 143) (end 139.541772 140.738993) (width 1) (layer "B.Cu") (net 29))
 (segment (start 150 137) (end 148 139) (width 1) (layer "B.Cu") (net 29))
 (segment (start 137.69 119.31) (end 139 118) (width 1) (layer "B.Cu") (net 29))
 (segment (start 148 139) (end 148 140) (width 1) (layer "B.Cu") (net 29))
 (segment (start 139 118) (end 147 118) (width 1) (layer "B.Cu") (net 29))
 (segment (start 137.69 121) (end 137.69 119.31) (width 1) (layer "B.Cu") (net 29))
 (segment (start 148 140) (end 145 143) (width 1) (layer "B.Cu") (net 29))
 (segment (start 124 66) (end 115 75) (width 1) (layer "B.Cu") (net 1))
 (segment (start 115 75) (end 115 89.125041) (width 1) (layer "B.Cu") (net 1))
 (segment (start 115 89.125041) (end 113.357863 90.767178) (width 1) (layer "B.Cu") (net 1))
 (segment (start 146.170001 63.110005) (end 143.280006 66) (width 1) (layer "B.Cu") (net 1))
 (segment (start 146.170001 63.110005) (end 151.230005 63.110005) (width 1) (layer "B.Cu") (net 1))
 (segment (start 143.280006 66) (end 124 66) (width 1) (layer "B.Cu") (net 1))
 (segment (start 151.230005 63.110005) (end 152.19 64.07) (width 1) (layer "B.Cu") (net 1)))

